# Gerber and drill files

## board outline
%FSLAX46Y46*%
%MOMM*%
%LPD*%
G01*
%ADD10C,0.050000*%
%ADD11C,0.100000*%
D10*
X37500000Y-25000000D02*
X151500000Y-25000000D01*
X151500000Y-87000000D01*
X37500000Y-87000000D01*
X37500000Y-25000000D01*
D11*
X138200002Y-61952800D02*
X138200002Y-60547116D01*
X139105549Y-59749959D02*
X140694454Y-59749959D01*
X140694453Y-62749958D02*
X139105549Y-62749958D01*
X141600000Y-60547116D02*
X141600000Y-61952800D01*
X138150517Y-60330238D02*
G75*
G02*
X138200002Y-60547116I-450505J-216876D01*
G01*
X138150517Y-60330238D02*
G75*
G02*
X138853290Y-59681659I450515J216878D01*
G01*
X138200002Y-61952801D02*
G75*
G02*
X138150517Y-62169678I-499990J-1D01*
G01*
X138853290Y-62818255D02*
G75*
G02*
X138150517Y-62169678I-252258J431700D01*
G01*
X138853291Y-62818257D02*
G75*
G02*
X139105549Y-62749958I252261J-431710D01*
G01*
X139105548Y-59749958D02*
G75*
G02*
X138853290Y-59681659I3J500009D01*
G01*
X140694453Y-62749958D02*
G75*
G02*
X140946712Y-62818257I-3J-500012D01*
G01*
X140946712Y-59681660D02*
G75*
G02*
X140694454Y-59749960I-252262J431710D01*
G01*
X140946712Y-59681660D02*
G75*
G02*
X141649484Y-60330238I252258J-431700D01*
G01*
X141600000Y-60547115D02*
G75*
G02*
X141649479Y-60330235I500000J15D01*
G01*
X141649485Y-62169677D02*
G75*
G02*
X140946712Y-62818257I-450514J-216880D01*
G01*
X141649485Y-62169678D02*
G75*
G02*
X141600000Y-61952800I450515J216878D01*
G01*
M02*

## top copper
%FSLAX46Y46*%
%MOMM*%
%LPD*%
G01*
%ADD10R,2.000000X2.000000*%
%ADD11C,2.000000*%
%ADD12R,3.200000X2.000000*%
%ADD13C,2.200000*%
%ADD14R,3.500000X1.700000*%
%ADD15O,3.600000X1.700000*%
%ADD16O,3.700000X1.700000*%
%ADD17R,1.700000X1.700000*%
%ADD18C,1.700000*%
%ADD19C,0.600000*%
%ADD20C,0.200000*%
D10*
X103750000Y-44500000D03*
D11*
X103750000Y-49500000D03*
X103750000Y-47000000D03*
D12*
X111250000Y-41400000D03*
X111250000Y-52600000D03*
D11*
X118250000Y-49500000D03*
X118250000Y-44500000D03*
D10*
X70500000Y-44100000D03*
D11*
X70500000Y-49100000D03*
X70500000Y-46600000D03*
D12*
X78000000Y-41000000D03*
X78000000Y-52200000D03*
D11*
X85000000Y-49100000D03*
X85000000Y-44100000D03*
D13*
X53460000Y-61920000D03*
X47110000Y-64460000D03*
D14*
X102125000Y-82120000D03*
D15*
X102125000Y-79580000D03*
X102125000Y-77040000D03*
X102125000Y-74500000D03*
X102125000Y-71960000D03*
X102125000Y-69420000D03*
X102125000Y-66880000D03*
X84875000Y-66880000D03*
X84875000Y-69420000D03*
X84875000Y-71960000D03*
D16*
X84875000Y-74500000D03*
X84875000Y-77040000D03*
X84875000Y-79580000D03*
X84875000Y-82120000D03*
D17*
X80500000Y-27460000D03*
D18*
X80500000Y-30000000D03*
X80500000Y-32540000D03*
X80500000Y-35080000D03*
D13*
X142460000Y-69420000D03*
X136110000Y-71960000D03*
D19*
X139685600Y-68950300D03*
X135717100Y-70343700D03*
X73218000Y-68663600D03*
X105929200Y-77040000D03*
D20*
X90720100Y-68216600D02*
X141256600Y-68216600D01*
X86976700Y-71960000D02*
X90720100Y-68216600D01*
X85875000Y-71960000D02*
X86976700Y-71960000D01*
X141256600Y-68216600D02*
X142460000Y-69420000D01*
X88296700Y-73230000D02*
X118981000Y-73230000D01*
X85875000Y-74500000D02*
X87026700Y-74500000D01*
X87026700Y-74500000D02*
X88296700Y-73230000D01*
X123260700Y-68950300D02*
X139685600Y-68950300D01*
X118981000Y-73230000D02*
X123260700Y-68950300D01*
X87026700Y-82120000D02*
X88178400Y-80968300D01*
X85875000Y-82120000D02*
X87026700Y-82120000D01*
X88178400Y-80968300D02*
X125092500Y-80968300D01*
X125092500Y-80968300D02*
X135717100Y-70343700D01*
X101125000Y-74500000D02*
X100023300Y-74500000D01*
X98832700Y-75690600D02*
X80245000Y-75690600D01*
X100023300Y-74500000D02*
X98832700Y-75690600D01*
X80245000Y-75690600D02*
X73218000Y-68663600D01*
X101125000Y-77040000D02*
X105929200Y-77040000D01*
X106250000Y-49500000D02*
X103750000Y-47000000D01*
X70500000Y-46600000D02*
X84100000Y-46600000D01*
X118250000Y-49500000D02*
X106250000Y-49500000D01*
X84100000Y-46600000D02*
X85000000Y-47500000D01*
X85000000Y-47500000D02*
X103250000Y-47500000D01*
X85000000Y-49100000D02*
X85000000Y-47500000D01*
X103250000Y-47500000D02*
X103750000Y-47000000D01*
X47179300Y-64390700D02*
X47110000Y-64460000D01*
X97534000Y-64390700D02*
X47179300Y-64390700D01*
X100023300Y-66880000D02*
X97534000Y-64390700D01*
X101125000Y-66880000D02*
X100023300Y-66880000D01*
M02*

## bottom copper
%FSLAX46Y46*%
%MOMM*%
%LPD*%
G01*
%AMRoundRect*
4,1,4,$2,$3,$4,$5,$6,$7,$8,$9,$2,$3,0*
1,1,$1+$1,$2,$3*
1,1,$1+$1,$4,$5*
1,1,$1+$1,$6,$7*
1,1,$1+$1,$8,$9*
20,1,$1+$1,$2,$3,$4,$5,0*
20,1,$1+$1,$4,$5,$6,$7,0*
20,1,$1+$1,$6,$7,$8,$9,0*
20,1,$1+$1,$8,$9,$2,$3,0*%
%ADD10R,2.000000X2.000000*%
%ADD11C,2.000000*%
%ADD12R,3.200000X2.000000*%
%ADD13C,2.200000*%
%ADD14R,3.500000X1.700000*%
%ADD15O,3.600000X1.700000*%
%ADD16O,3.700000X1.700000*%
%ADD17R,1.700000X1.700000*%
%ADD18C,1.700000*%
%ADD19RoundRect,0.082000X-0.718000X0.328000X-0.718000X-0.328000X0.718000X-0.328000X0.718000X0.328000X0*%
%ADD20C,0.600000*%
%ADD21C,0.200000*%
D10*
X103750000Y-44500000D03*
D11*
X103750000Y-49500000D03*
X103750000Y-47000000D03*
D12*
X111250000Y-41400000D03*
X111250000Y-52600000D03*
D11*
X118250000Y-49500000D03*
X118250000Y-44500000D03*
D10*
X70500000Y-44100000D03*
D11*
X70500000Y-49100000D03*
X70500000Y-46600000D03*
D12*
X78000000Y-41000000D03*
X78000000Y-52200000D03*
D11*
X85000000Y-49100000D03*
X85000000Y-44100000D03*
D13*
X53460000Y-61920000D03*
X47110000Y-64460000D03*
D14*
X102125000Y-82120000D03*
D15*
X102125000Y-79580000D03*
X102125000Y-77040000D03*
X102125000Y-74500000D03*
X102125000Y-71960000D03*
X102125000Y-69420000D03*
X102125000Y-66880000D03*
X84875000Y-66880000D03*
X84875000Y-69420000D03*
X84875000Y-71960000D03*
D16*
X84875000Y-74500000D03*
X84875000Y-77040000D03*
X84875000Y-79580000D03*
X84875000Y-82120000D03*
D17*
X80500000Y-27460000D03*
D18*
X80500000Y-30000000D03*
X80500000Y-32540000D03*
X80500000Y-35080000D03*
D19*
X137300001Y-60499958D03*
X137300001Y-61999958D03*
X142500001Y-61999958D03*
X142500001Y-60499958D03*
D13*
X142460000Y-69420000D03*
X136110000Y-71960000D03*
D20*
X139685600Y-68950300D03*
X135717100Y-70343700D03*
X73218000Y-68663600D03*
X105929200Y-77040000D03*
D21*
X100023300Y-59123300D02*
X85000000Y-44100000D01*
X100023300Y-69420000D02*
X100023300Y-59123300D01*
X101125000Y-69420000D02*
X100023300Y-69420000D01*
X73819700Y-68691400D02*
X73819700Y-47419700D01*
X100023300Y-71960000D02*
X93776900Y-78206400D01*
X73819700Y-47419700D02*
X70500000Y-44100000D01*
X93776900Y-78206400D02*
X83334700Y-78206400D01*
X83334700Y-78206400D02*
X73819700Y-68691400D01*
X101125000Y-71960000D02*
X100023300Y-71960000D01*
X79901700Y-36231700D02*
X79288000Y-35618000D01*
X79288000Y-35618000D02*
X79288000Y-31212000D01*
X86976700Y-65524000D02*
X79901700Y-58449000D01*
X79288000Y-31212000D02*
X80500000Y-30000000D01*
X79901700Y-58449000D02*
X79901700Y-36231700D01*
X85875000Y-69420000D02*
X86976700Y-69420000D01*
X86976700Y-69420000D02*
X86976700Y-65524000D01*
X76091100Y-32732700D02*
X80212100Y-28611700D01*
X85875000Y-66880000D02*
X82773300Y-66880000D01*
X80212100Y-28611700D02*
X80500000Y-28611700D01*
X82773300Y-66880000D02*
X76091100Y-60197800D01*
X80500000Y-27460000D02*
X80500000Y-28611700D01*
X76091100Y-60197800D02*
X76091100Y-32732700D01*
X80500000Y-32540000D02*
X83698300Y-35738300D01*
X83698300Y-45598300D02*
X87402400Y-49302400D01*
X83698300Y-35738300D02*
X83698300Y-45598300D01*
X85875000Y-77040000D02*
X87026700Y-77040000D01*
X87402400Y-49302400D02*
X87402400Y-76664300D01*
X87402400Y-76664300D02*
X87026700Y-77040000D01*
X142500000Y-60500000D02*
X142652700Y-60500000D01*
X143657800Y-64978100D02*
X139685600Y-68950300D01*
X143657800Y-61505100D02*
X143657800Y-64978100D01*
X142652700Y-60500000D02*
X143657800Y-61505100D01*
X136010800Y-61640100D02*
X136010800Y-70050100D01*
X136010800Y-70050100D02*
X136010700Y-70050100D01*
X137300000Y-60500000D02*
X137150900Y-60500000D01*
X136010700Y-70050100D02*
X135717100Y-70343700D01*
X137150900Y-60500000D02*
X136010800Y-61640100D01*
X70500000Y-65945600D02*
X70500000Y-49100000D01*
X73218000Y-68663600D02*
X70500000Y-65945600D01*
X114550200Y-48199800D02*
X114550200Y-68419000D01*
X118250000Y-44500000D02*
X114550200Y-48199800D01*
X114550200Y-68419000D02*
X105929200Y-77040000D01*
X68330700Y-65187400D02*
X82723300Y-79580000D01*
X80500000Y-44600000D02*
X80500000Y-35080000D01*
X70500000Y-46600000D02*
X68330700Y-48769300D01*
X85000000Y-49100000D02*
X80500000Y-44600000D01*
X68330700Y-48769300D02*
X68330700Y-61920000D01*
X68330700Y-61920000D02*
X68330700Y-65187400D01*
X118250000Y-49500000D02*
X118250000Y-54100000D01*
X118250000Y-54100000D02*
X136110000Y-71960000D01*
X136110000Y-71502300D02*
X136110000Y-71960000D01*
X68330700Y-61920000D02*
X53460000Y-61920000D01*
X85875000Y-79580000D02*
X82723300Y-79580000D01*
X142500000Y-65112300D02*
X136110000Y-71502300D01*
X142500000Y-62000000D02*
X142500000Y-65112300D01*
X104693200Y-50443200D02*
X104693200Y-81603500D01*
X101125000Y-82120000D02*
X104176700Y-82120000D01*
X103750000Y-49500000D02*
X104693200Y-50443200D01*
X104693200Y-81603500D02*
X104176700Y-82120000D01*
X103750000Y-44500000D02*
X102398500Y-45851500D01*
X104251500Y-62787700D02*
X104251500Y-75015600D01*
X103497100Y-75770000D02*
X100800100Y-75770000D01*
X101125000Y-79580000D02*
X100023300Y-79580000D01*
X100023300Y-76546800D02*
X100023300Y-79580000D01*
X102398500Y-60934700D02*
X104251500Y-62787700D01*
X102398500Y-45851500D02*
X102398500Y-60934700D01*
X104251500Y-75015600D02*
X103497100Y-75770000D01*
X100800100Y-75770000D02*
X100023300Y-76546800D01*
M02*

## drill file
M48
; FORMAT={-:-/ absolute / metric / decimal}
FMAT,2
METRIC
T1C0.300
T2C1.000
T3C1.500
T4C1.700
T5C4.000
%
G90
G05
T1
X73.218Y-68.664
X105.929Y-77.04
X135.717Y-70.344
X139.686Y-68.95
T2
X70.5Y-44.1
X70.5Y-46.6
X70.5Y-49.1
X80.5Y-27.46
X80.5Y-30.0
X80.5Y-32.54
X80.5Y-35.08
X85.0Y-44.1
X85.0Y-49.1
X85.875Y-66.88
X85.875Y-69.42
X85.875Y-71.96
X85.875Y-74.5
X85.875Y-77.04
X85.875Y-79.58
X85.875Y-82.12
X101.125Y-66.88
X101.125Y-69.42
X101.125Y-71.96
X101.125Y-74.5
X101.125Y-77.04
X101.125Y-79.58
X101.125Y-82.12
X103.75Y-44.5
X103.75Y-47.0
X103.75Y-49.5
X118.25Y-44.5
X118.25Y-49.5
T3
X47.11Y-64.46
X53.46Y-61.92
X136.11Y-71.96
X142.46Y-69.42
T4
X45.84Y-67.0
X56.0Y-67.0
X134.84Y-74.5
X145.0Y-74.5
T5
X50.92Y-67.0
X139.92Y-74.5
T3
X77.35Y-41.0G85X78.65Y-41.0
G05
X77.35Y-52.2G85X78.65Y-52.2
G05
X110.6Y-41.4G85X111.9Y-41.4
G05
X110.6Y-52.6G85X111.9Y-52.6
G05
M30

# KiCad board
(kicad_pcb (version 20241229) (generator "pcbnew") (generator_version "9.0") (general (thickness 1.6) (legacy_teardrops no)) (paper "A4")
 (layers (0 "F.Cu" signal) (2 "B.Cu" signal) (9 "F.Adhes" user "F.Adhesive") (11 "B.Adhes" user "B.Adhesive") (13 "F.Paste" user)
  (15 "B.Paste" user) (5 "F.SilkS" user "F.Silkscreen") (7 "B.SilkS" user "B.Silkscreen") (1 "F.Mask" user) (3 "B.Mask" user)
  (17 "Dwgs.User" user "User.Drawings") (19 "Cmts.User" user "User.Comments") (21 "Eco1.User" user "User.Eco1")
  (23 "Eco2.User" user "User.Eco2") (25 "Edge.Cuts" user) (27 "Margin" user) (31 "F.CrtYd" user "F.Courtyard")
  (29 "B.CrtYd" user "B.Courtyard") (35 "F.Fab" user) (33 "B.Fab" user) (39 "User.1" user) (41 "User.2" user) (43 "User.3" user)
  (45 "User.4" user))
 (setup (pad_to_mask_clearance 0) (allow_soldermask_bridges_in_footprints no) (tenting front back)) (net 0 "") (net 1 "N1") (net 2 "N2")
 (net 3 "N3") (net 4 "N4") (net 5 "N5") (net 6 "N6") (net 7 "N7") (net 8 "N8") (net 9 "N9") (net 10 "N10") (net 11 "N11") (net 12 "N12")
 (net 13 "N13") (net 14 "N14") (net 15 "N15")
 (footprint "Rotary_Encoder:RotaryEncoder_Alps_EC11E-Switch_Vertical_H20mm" (layer "F.Cu") (at 103.75 44.5)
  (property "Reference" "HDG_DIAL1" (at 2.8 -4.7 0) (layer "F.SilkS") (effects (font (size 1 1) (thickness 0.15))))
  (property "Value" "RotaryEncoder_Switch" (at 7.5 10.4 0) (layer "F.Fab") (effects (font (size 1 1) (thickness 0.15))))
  (pad "A" thru_hole rect (at 0 0) (size 2 2) (drill 1) (layers "*.Cu" "*.Mask") (remove_unused_layers no) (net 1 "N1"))
  (pad "B" thru_hole circle (at 0 5) (size 2 2) (drill 1) (layers "*.Cu" "*.Mask") (remove_unused_layers no) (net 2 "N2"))
  (pad "C" thru_hole circle (at 0 2.5) (size 2 2) (drill 1) (layers "*.Cu" "*.Mask") (remove_unused_layers no) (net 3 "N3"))
  (pad "MP" thru_hole rect (at 7.5 -3.1) (size 3.2 2) (drill oval 2.8 1.5) (layers "*.Cu" "*.Mask") (remove_unused_layers no))
  (pad "MP" thru_hole rect (at 7.5 8.1) (size 3.2 2) (drill oval 2.8 1.5) (layers "*.Cu" "*.Mask") (remove_unused_layers no))
  (pad "S1" thru_hole circle (at 14.5 5) (size 2 2) (drill 1) (layers "*.Cu" "*.Mask") (remove_unused_layers no) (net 3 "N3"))
  (pad "S2" thru_hole circle (at 14.5 0) (size 2 2) (drill 1) (layers "*.Cu" "*.Mask") (remove_unused_layers no) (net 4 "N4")))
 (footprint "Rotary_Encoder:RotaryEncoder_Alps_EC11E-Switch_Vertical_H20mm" (layer "F.Cu") (at 70.5 44.1)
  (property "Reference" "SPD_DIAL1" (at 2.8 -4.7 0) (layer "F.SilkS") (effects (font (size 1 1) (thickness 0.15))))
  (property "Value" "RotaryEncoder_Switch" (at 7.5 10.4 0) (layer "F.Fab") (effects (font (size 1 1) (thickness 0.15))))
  (pad "A" thru_hole rect (at 0 0) (size 2 2) (drill 1) (layers "*.Cu" "*.Mask") (remove_unused_layers no) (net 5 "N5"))
  (pad "B" thru_hole circle (at 0 5) (size 2 2) (drill 1) (layers "*.Cu" "*.Mask") (remove_unused_layers no) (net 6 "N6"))
  (pad "C" thru_hole circle (at 0 2.5) (size 2 2) (drill 1) (layers "*.Cu" "*.Mask") (remove_unused_layers no) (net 3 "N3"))
  (pad "MP" thru_hole rect (at 7.5 -3.1) (size 3.2 2) (drill oval 2.8 1.5) (layers "*.Cu" "*.Mask") (remove_unused_layers no))
  (pad "MP" thru_hole rect (at 7.5 8.1) (size 3.2 2) (drill oval 2.8 1.5) (layers "*.Cu" "*.Mask") (remove_unused_layers no))
  (pad "S1" thru_hole circle (at 14.5 5) (size 2 2) (drill 1) (layers "*.Cu" "*.Mask") (remove_unused_layers no) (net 3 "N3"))
  (pad "S2" thru_hole circle (at 14.5 0) (size 2 2) (drill 1) (layers "*.Cu" "*.Mask") (remove_unused_layers no) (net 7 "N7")))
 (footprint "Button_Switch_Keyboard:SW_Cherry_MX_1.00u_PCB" (layer "F.Cu") (at 53.46 61.92)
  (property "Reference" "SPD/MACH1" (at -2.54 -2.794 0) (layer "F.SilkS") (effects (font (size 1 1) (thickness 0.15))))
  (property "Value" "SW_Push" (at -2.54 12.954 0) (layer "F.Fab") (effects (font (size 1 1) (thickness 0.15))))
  (pad "" np_thru_hole circle (at -7.62 5.08) (size 1.7 1.7) (drill 1.7) (layers "*.Cu" "*.Mask"))
  (pad "" np_thru_hole circle (at -2.54 5.08) (size 4 4) (drill 4) (layers "*.Cu" "*.Mask"))
  (pad "" np_thru_hole circle (at 2.54 5.08) (size 1.7 1.7) (drill 1.7) (layers "*.Cu" "*.Mask"))
  (pad "1" thru_hole circle (at 0 0) (size 2.2 2.2) (drill 1.5) (layers "*.Cu" "*.Mask") (remove_unused_layers no) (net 3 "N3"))
  (pad "2" thru_hole circle (at -6.35 2.54) (size 2.2 2.2) (drill 1.5) (layers "*.Cu" "*.Mask") (remove_unused_layers no) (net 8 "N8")))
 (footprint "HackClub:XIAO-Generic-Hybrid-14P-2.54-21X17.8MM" (layer "F.Cu") (at 93.5 74.5 180)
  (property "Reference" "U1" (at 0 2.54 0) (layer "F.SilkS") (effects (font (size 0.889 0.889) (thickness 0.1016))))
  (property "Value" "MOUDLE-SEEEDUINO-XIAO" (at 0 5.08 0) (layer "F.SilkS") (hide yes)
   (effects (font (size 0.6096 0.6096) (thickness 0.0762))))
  (pad "1" thru_hole rect (at -7.625 -7.62 180) (size 3.5 1.7) (drill 1 (offset -1 0)) (layers "*.Cu" "*.Mask") (remove_unused_layers no)
   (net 2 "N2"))
  (pad "2" thru_hole oval (at -7.625 -5.08 180) (size 3.6 1.7) (drill 1 (offset -1 0)) (layers "*.Cu" "*.Mask") (remove_unused_layers no)
   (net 1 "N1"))
  (pad "3" thru_hole oval (at -7.625 -2.54 180) (size 3.6 1.7) (drill 1 (offset -1 0)) (layers "*.Cu" "*.Mask") (remove_unused_layers no)
   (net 4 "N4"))
  (pad "4" thru_hole oval (at -7.625 0 180) (size 3.6 1.7) (drill 1 (offset -1 0)) (layers "*.Cu" "*.Mask") (remove_unused_layers no)
   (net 6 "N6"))
  (pad "5" thru_hole oval (at -7.625 2.54 180) (size 3.6 1.7) (drill 1 (offset -1 0)) (layers "*.Cu" "*.Mask") (remove_unused_layers no)
   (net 5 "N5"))
  (pad "6" thru_hole oval (at -7.625 5.08) (size 3.6 1.7) (drill 1 (offset 1 0)) (layers "*.Cu" "*.Mask") (remove_unused_layers no)
   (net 7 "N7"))
  (pad "7" thru_hole oval (at -7.625 7.62 180) (size 3.6 1.7) (drill 1 (offset -1 0)) (layers "*.Cu" "*.Mask") (remove_unused_layers no)
   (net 8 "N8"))
  (pad "8" thru_hole oval (at 7.625 7.62 180) (size 3.6 1.7) (drill 1 (offset 1 0)) (layers "*.Cu" "*.Mask") (remove_unused_layers no)
   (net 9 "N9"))
  (pad "9" thru_hole oval (at 7.625 5.08 180) (size 3.6 1.7) (drill 1 (offset 1 0)) (layers "*.Cu" "*.Mask") (remove_unused_layers no)
   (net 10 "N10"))
  (pad "10" thru_hole oval (at 7.625 2.54 180) (size 3.6 1.7) (drill 1 (offset 1 0)) (layers "*.Cu" "*.Mask") (remove_unused_layers no)
   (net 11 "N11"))
  (pad "11" thru_hole oval (at 7.625 0 180) (size 3.7 1.7) (drill 1 (offset 1 0)) (layers "*.Cu" "*.Mask") (remove_unused_layers no)
   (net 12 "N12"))
  (pad "12" thru_hole oval (at 7.625 -2.54 180) (size 3.7 1.7) (drill 1 (offset 1 0)) (layers "*.Cu" "*.Mask") (remove_unused_layers no)
   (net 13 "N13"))
  (pad "13" thru_hole oval (at 7.625 -5.08 180) (size 3.7 1.7) (drill 1 (offset 1 0)) (layers "*.Cu" "*.Mask") (remove_unused_layers no)
   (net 3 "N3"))
  (pad "14" thru_hole oval (at 7.625 -7.62 180) (size 3.7 1.7) (drill 1 (offset 1 0)) (layers "*.Cu" "*.Mask") (remove_unused_layers no)
   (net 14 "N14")))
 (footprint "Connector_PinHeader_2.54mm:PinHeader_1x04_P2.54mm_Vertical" (layer "F.Cu") (at 80.5 27.46)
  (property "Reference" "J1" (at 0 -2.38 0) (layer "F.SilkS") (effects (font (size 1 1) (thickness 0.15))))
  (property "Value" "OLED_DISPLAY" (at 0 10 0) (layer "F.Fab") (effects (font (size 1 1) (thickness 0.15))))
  (pad "1" thru_hole rect (at 0 0) (size 1.7 1.7) (drill 1) (layers "*.Cu" "*.Mask") (remove_unused_layers no) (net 9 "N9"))
  (pad "2" thru_hole circle (at 0 2.54) (size 1.7 1.7) (drill 1) (layers "*.Cu" "*.Mask") (remove_unused_layers no) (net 10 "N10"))
  (pad "3" thru_hole circle (at 0 5.08) (size 1.7 1.7) (drill 1) (layers "*.Cu" "*.Mask") (remove_unused_layers no) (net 13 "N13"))
  (pad "4" thru_hole circle (at 0 7.62) (size 1.7 1.7) (drill 1) (layers "*.Cu" "*.Mask") (remove_unused_layers no) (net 3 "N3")))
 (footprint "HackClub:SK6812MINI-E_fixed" (layer "F.Cu") (at 139.9 61.3528)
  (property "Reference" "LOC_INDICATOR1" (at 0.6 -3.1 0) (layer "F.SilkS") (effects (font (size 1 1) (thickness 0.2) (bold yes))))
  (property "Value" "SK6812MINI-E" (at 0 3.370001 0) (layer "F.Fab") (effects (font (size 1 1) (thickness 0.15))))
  (fp_line (start -1.699998 0.6) (end -1.699998 -0.805684) (stroke (width 0.1) (type solid)) (layer "Edge.Cuts"))
  (fp_line (start -0.794451 -1.602841) (end 0.794454 -1.602841) (stroke (width 0.1) (type solid)) (layer "Edge.Cuts"))
  (fp_line (start 0.794453 1.397158) (end -0.794451 1.397158) (stroke (width 0.1) (type solid)) (layer "Edge.Cuts"))
  (fp_line (start 1.7 -0.805684) (end 1.7 0.6) (stroke (width 0.1) (type solid)) (layer "Edge.Cuts"))
  (fp_arc (start -1.749483 -1.022562) (mid -1.712526 -0.91691) (end -1.699998 -0.805684) (stroke (width 0.1) (type solid))
   (layer "Edge.Cuts"))
  (fp_arc (start -1.749483 -1.022562) (mid -1.63807 -1.606877) (end -1.04671 -1.671141) (stroke (width 0.1) (type solid))
   (layer "Edge.Cuts"))
  (fp_arc (start -1.699998 0.600001) (mid -1.712526 0.711226) (end -1.749483 0.816878) (stroke (width 0.1) (type solid)) (layer "Edge.Cuts"))
  (fp_arc (start -1.04671 1.465455) (mid -1.638069 1.401192) (end -1.749483 0.816878) (stroke (width 0.1) (type solid)) (layer "Edge.Cuts"))
  (fp_arc (start -1.046709 1.465457) (mid -0.925121 1.414535) (end -0.794451 1.397158) (stroke (width 0.1) (type solid)) (layer "Edge.Cuts"))
  (fp_arc (start -0.794452 -1.602842) (mid -0.925122 -1.620219) (end -1.04671 -1.671141) (stroke (width 0.1) (type solid))
   (layer "Edge.Cuts"))
  (fp_arc (start 0.794453 1.397158) (mid 0.925124 1.414535) (end 1.046712 1.465457) (stroke (width 0.1) (type solid)) (layer "Edge.Cuts"))
  (fp_arc (start 1.046712 -1.67114) (mid 0.925124 -1.620218) (end 0.794454 -1.602841) (stroke (width 0.1) (type solid)) (layer "Edge.Cuts"))
  (fp_arc (start 1.046712 -1.67114) (mid 1.638072 -1.606876) (end 1.749485 -1.022562) (stroke (width 0.1) (type solid)) (layer "Edge.Cuts"))
  (fp_arc (start 1.7 -0.805685) (mid 1.712528 -0.91691) (end 1.749485 -1.022562) (stroke (width 0.1) (type solid)) (layer "Edge.Cuts"))
  (fp_arc (start 1.749485 0.816877) (mid 1.638073 1.401193) (end 1.046712 1.465457) (stroke (width 0.1) (type solid)) (layer "Edge.Cuts"))
  (fp_arc (start 1.749485 0.816878) (mid 1.712528 0.711226) (end 1.7 0.6) (stroke (width 0.1) (type solid)) (layer "Edge.Cuts"))
  (pad "1" smd roundrect (at -2.599999 -0.852842 270) (size 0.82 1.6) (layers "B.Cu" "B.Mask" "B.Paste") (roundrect_rratio 0.1)
   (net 14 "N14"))
  (pad "2" smd roundrect (at -2.599999 0.647158 270) (size 0.82 1.6) (layers "B.Cu" "B.Mask" "B.Paste") (roundrect_rratio 0.1)
   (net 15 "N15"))
  (pad "3" smd roundrect (at 2.600001 0.647158 270) (size 0.82 1.6) (layers "B.Cu" "B.Mask" "B.Paste") (roundrect_rratio 0.1) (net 3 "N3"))
  (pad "4" smd roundrect (at 2.600001 -0.852842 270) (size 0.82 1.6) (layers "B.Cu" "B.Mask" "B.Paste") (roundrect_rratio 0.1)
   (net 12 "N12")))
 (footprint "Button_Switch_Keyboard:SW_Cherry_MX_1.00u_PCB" (layer "F.Cu") (at 142.46 69.42)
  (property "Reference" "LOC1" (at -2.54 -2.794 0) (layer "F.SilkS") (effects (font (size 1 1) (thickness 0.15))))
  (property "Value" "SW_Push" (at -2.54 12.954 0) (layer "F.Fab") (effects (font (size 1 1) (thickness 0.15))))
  (pad "" np_thru_hole circle (at -7.62 5.08) (size 1.7 1.7) (drill 1.7) (layers "*.Cu" "*.Mask"))
  (pad "" np_thru_hole circle (at -2.54 5.08) (size 4 4) (drill 4) (layers "*.Cu" "*.Mask"))
  (pad "" np_thru_hole circle (at 2.54 5.08) (size 1.7 1.7) (drill 1.7) (layers "*.Cu" "*.Mask"))
  (pad "1" thru_hole circle (at 0 0) (size 2.2 2.2) (drill 1.5) (layers "*.Cu" "*.Mask") (remove_unused_layers no) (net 11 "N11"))
  (pad "2" thru_hole circle (at -6.35 2.54) (size 2.2 2.2) (drill 1.5) (layers "*.Cu" "*.Mask") (remove_unused_layers no) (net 3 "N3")))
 (gr_rect (start 37.5 25) (end 151.5 87) (stroke (width 0.05) (type default)) (fill no) (layer "Edge.Cuts"))
 (segment (start 100.0233 59.1233) (end 85 44.1) (width 0.2) (layer "B.Cu") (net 7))
 (segment (start 100.0233 69.42) (end 100.0233 59.1233) (width 0.2) (layer "B.Cu") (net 7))
 (segment (start 101.125 69.42) (end 100.0233 69.42) (width 0.2) (layer "B.Cu") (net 7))
 (segment (start 73.8197 68.6914) (end 73.8197 47.4197) (width 0.2) (layer "B.Cu") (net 5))
 (segment (start 100.0233 71.96) (end 93.7769 78.2064) (width 0.2) (layer "B.Cu") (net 5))
 (segment (start 73.8197 47.4197) (end 70.5 44.1) (width 0.2) (layer "B.Cu") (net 5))
 (segment (start 93.7769 78.2064) (end 83.3347 78.2064) (width 0.2) (layer "B.Cu") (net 5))
 (segment (start 83.3347 78.2064) (end 73.8197 68.6914) (width 0.2) (layer "B.Cu") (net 5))
 (segment (start 101.125 71.96) (end 100.0233 71.96) (width 0.2) (layer "B.Cu") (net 5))
 (segment (start 79.9017 36.2317) (end 79.288 35.618) (width 0.2) (layer "B.Cu") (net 10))
 (segment (start 79.288 35.618) (end 79.288 31.212) (width 0.2) (layer "B.Cu") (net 10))
 (segment (start 86.9767 65.524) (end 79.9017 58.449) (width 0.2) (layer "B.Cu") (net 10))
 (segment (start 79.288 31.212) (end 80.5 30) (width 0.2) (layer "B.Cu") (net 10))
 (segment (start 79.9017 58.449) (end 79.9017 36.2317) (width 0.2) (layer "B.Cu") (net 10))
 (segment (start 85.875 69.42) (end 86.9767 69.42) (width 0.2) (layer "B.Cu") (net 10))
 (segment (start 86.9767 69.42) (end 86.9767 65.524) (width 0.2) (layer "B.Cu") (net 10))
 (segment (start 76.0911 32.7327) (end 80.2121 28.6117) (width 0.2) (layer "B.Cu") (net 9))
 (segment (start 85.875 66.88) (end 82.7733 66.88) (width 0.2) (layer "B.Cu") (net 9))
 (segment (start 80.2121 28.6117) (end 80.5 28.6117) (width 0.2) (layer "B.Cu") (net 9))
 (segment (start 82.7733 66.88) (end 76.0911 60.1978) (width 0.2) (layer "B.Cu") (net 9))
 (segment (start 80.5 27.46) (end 80.5 28.6117) (width 0.2) (layer "B.Cu") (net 9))
 (segment (start 76.0911 60.1978) (end 76.0911 32.7327) (width 0.2) (layer "B.Cu") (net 9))
 (segment (start 80.5 32.54) (end 83.6983 35.7383) (width 0.2) (layer "B.Cu") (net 13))
 (segment (start 83.6983 45.5983) (end 87.4024 49.3024) (width 0.2) (layer "B.Cu") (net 13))
 (segment (start 83.6983 35.7383) (end 83.6983 45.5983) (width 0.2) (layer "B.Cu") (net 13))
 (segment (start 85.875 77.04) (end 87.0267 77.04) (width 0.2) (layer "B.Cu") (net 13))
 (segment (start 87.4024 49.3024) (end 87.4024 76.6643) (width 0.2) (layer "B.Cu") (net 13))
 (segment (start 87.4024 76.6643) (end 87.0267 77.04) (width 0.2) (layer "B.Cu") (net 13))
 (segment (start 90.7201 68.2166) (end 141.2566 68.2166) (width 0.2) (layer "F.Cu") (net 11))
 (segment (start 86.9767 71.96) (end 90.7201 68.2166) (width 0.2) (layer "F.Cu") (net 11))
 (segment (start 85.875 71.96) (end 86.9767 71.96) (width 0.2) (layer "F.Cu") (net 11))
 (segment (start 141.2566 68.2166) (end 142.46 69.42) (width 0.2) (layer "F.Cu") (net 11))
 (segment (start 88.2967 73.23) (end 118.981 73.23) (width 0.2) (layer "F.Cu") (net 12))
 (segment (start 85.875 74.5) (end 87.0267 74.5) (width 0.2) (layer "F.Cu") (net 12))
 (segment (start 87.0267 74.5) (end 88.2967 73.23) (width 0.2) (layer "F.Cu") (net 12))
 (segment (start 123.2607 68.9503) (end 139.6856 68.9503) (width 0.2) (layer "F.Cu") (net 12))
 (segment (start 118.981 73.23) (end 123.2607 68.9503) (width 0.2) (layer "F.Cu") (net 12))
 (via (at 139.6856 68.9503) (size 0.6) (drill 0.3) (layers "F.Cu" "B.Cu") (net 12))
 (segment (start 142.5 60.5) (end 142.6527 60.5) (width 0.2) (layer "B.Cu") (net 12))
 (segment (start 143.6578 64.9781) (end 139.6856 68.9503) (width 0.2) (layer "B.Cu") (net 12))
 (segment (start 143.6578 61.5051) (end 143.6578 64.9781) (width 0.2) (layer "B.Cu") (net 12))
 (segment (start 142.6527 60.5) (end 143.6578 61.5051) (width 0.2) (layer "B.Cu") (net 12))
 (segment (start 87.0267 82.12) (end 88.1784 80.9683) (width 0.2) (layer "F.Cu") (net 14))
 (segment (start 85.875 82.12) (end 87.0267 82.12) (width 0.2) (layer "F.Cu") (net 14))
 (segment (start 88.1784 80.9683) (end 125.0925 80.9683) (width 0.2) (layer "F.Cu") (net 14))
 (segment (start 125.0925 80.9683) (end 135.7171 70.3437) (width 0.2) (layer "F.Cu") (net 14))
 (via (at 135.7171 70.3437) (size 0.6) (drill 0.3) (layers "F.Cu" "B.Cu") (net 14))
 (segment (start 136.0108 61.6401) (end 136.0108 70.0501) (width 0.2) (layer "B.Cu") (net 14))
 (segment (start 136.0108 70.0501) (end 136.0107 70.0501) (width 0.2) (layer "B.Cu") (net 14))
 (segment (start 137.3 60.5) (end 137.1509 60.5) (width 0.2) (layer "B.Cu") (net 14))
 (segment (start 136.0107 70.0501) (end 135.7171 70.3437) (width 0.2) (layer "B.Cu") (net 14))
 (segment (start 137.1509 60.5) (end 136.0108 61.6401) (width 0.2) (layer "B.Cu") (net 14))
 (segment (start 101.125 74.5) (end 100.0233 74.5) (width 0.2) (layer "F.Cu") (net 6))
 (segment (start 98.8327 75.6906) (end 80.245 75.6906) (width 0.2) (layer "F.Cu") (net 6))
 (segment (start 100.0233 74.5) (end 98.8327 75.6906) (width 0.2) (layer "F.Cu") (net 6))
 (segment (start 80.245 75.6906) (end 73.218 68.6636) (width 0.2) (layer "F.Cu") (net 6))
 (via (at 73.218 68.6636) (size 0.6) (drill 0.3) (layers "F.Cu" "B.Cu") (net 6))
 (segment (start 70.5 65.9456) (end 70.5 49.1) (width 0.2) (layer "B.Cu") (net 6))
 (segment (start 73.218 68.6636) (end 70.5 65.9456) (width 0.2) (layer "B.Cu") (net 6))
 (segment (start 101.125 77.04) (end 105.9292 77.04) (width 0.2) (layer "F.Cu") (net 4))
 (via (at 105.9292 77.04) (size 0.6) (drill 0.3) (layers "F.Cu" "B.Cu") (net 4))
 (segment (start 114.5502 48.1998) (end 114.5502 68.419) (width 0.2) (layer "B.Cu") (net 4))
 (segment (start 118.25 44.5) (end 114.5502 48.1998) (width 0.2) (layer "B.Cu") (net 4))
 (segment (start 114.5502 68.419) (end 105.9292 77.04) (width 0.2) (layer "B.Cu") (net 4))
 (segment (start 106.25 49.5) (end 103.75 47) (width 0.2) (layer "F.Cu") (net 3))
 (segment (start 70.5 46.6) (end 84.1 46.6) (width 0.2) (layer "F.Cu") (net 3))
 (segment (start 118.25 49.5) (end 106.25 49.5) (width 0.2) (layer "F.Cu") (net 3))
 (segment (start 84.1 46.6) (end 85 47.5) (width 0.2) (layer "F.Cu") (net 3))
 (segment (start 85 47.5) (end 103.25 47.5) (width 0.2) (layer "F.Cu") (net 3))
 (segment (start 85 49.1) (end 85 47.5) (width 0.2) (layer "F.Cu") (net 3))
 (segment (start 103.25 47.5) (end 103.75 47) (width 0.2) (layer "F.Cu") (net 3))
 (segment (start 68.3307 65.1874) (end 82.7233 79.58) (width 0.2) (layer "B.Cu") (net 3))
 (segment (start 80.5 44.6) (end 80.5 35.08) (width 0.2) (layer "B.Cu") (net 3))
 (segment (start 70.5 46.6) (end 68.3307 48.7693) (width 0.2) (layer "B.Cu") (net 3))
 (segment (start 85 49.1) (end 80.5 44.6) (width 0.2) (layer "B.Cu") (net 3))
 (segment (start 68.3307 48.7693) (end 68.3307 61.92) (width 0.2) (layer "B.Cu") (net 3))
 (segment (start 68.3307 61.92) (end 68.3307 65.1874) (width 0.2) (layer "B.Cu") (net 3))
 (segment (start 118.25 49.5) (end 118.25 54.1) (width 0.2) (layer "B.Cu") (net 3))
 (segment (start 118.25 54.1) (end 136.11 71.96) (width 0.2) (layer "B.Cu") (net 3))
 (segment (start 136.11 71.5023) (end 136.11 71.96) (width 0.2) (layer "B.Cu") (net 3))
 (segment (start 68.3307 61.92) (end 53.46 61.92) (width 0.2) (layer "B.Cu") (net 3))
 (segment (start 85.875 79.58) (end 82.7233 79.58) (width 0.2) (layer "B.Cu") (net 3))
 (segment (start 142.5 65.1123) (end 136.11 71.5023) (width 0.2) (layer "B.Cu") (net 3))
 (segment (start 142.5 62) (end 142.5 65.1123) (width 0.2) (layer "B.Cu") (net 3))
 (segment (start 104.6932 50.4432) (end 104.6932 81.6035) (width 0.2) (layer "B.Cu") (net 2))
 (segment (start 101.125 82.12) (end 104.1767 82.12) (width 0.2) (layer "B.Cu") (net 2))
 (segment (start 103.75 49.5) (end 104.6932 50.4432) (width 0.2) (layer "B.Cu") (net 2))
 (segment (start 104.6932 81.6035) (end 104.1767 82.12) (width 0.2) (layer "B.Cu") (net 2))
 (segment (start 103.75 44.5) (end 102.3985 45.8515) (width 0.2) (layer "B.Cu") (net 1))
 (segment (start 104.2515 62.7877) (end 104.2515 75.0156) (width 0.2) (layer "B.Cu") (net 1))
 (segment (start 103.4971 75.77) (end 100.8001 75.77) (width 0.2) (layer "B.Cu") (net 1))
 (segment (start 101.125 79.58) (end 100.0233 79.58) (width 0.2) (layer "B.Cu") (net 1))
 (segment (start 100.0233 76.5468) (end 100.0233 79.58) (width 0.2) (layer "B.Cu") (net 1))
 (segment (start 102.3985 60.9347) (end 104.2515 62.7877) (width 0.2) (layer "B.Cu") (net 1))
 (segment (start 102.3985 45.8515) (end 102.3985 60.9347) (width 0.2) (layer "B.Cu") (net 1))
 (segment (start 104.2515 75.0156) (end 103.4971 75.77) (width 0.2) (layer "B.Cu") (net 1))
 (segment (start 100.8001 75.77) (end 100.0233 76.5468) (width 0.2) (layer "B.Cu") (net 1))
 (segment (start 47.1793 64.3907) (end 47.11 64.46) (width 0.2) (layer "F.Cu") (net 8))
 (segment (start 97.534 64.3907) (end 47.1793 64.3907) (width 0.2) (layer "F.Cu") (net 8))
 (segment (start 100.0233 66.88) (end 97.534 64.3907) (width 0.2) (layer "F.Cu") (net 8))
 (segment (start 101.125 66.88) (end 100.0233 66.88) (width 0.2) (layer "F.Cu") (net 8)))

